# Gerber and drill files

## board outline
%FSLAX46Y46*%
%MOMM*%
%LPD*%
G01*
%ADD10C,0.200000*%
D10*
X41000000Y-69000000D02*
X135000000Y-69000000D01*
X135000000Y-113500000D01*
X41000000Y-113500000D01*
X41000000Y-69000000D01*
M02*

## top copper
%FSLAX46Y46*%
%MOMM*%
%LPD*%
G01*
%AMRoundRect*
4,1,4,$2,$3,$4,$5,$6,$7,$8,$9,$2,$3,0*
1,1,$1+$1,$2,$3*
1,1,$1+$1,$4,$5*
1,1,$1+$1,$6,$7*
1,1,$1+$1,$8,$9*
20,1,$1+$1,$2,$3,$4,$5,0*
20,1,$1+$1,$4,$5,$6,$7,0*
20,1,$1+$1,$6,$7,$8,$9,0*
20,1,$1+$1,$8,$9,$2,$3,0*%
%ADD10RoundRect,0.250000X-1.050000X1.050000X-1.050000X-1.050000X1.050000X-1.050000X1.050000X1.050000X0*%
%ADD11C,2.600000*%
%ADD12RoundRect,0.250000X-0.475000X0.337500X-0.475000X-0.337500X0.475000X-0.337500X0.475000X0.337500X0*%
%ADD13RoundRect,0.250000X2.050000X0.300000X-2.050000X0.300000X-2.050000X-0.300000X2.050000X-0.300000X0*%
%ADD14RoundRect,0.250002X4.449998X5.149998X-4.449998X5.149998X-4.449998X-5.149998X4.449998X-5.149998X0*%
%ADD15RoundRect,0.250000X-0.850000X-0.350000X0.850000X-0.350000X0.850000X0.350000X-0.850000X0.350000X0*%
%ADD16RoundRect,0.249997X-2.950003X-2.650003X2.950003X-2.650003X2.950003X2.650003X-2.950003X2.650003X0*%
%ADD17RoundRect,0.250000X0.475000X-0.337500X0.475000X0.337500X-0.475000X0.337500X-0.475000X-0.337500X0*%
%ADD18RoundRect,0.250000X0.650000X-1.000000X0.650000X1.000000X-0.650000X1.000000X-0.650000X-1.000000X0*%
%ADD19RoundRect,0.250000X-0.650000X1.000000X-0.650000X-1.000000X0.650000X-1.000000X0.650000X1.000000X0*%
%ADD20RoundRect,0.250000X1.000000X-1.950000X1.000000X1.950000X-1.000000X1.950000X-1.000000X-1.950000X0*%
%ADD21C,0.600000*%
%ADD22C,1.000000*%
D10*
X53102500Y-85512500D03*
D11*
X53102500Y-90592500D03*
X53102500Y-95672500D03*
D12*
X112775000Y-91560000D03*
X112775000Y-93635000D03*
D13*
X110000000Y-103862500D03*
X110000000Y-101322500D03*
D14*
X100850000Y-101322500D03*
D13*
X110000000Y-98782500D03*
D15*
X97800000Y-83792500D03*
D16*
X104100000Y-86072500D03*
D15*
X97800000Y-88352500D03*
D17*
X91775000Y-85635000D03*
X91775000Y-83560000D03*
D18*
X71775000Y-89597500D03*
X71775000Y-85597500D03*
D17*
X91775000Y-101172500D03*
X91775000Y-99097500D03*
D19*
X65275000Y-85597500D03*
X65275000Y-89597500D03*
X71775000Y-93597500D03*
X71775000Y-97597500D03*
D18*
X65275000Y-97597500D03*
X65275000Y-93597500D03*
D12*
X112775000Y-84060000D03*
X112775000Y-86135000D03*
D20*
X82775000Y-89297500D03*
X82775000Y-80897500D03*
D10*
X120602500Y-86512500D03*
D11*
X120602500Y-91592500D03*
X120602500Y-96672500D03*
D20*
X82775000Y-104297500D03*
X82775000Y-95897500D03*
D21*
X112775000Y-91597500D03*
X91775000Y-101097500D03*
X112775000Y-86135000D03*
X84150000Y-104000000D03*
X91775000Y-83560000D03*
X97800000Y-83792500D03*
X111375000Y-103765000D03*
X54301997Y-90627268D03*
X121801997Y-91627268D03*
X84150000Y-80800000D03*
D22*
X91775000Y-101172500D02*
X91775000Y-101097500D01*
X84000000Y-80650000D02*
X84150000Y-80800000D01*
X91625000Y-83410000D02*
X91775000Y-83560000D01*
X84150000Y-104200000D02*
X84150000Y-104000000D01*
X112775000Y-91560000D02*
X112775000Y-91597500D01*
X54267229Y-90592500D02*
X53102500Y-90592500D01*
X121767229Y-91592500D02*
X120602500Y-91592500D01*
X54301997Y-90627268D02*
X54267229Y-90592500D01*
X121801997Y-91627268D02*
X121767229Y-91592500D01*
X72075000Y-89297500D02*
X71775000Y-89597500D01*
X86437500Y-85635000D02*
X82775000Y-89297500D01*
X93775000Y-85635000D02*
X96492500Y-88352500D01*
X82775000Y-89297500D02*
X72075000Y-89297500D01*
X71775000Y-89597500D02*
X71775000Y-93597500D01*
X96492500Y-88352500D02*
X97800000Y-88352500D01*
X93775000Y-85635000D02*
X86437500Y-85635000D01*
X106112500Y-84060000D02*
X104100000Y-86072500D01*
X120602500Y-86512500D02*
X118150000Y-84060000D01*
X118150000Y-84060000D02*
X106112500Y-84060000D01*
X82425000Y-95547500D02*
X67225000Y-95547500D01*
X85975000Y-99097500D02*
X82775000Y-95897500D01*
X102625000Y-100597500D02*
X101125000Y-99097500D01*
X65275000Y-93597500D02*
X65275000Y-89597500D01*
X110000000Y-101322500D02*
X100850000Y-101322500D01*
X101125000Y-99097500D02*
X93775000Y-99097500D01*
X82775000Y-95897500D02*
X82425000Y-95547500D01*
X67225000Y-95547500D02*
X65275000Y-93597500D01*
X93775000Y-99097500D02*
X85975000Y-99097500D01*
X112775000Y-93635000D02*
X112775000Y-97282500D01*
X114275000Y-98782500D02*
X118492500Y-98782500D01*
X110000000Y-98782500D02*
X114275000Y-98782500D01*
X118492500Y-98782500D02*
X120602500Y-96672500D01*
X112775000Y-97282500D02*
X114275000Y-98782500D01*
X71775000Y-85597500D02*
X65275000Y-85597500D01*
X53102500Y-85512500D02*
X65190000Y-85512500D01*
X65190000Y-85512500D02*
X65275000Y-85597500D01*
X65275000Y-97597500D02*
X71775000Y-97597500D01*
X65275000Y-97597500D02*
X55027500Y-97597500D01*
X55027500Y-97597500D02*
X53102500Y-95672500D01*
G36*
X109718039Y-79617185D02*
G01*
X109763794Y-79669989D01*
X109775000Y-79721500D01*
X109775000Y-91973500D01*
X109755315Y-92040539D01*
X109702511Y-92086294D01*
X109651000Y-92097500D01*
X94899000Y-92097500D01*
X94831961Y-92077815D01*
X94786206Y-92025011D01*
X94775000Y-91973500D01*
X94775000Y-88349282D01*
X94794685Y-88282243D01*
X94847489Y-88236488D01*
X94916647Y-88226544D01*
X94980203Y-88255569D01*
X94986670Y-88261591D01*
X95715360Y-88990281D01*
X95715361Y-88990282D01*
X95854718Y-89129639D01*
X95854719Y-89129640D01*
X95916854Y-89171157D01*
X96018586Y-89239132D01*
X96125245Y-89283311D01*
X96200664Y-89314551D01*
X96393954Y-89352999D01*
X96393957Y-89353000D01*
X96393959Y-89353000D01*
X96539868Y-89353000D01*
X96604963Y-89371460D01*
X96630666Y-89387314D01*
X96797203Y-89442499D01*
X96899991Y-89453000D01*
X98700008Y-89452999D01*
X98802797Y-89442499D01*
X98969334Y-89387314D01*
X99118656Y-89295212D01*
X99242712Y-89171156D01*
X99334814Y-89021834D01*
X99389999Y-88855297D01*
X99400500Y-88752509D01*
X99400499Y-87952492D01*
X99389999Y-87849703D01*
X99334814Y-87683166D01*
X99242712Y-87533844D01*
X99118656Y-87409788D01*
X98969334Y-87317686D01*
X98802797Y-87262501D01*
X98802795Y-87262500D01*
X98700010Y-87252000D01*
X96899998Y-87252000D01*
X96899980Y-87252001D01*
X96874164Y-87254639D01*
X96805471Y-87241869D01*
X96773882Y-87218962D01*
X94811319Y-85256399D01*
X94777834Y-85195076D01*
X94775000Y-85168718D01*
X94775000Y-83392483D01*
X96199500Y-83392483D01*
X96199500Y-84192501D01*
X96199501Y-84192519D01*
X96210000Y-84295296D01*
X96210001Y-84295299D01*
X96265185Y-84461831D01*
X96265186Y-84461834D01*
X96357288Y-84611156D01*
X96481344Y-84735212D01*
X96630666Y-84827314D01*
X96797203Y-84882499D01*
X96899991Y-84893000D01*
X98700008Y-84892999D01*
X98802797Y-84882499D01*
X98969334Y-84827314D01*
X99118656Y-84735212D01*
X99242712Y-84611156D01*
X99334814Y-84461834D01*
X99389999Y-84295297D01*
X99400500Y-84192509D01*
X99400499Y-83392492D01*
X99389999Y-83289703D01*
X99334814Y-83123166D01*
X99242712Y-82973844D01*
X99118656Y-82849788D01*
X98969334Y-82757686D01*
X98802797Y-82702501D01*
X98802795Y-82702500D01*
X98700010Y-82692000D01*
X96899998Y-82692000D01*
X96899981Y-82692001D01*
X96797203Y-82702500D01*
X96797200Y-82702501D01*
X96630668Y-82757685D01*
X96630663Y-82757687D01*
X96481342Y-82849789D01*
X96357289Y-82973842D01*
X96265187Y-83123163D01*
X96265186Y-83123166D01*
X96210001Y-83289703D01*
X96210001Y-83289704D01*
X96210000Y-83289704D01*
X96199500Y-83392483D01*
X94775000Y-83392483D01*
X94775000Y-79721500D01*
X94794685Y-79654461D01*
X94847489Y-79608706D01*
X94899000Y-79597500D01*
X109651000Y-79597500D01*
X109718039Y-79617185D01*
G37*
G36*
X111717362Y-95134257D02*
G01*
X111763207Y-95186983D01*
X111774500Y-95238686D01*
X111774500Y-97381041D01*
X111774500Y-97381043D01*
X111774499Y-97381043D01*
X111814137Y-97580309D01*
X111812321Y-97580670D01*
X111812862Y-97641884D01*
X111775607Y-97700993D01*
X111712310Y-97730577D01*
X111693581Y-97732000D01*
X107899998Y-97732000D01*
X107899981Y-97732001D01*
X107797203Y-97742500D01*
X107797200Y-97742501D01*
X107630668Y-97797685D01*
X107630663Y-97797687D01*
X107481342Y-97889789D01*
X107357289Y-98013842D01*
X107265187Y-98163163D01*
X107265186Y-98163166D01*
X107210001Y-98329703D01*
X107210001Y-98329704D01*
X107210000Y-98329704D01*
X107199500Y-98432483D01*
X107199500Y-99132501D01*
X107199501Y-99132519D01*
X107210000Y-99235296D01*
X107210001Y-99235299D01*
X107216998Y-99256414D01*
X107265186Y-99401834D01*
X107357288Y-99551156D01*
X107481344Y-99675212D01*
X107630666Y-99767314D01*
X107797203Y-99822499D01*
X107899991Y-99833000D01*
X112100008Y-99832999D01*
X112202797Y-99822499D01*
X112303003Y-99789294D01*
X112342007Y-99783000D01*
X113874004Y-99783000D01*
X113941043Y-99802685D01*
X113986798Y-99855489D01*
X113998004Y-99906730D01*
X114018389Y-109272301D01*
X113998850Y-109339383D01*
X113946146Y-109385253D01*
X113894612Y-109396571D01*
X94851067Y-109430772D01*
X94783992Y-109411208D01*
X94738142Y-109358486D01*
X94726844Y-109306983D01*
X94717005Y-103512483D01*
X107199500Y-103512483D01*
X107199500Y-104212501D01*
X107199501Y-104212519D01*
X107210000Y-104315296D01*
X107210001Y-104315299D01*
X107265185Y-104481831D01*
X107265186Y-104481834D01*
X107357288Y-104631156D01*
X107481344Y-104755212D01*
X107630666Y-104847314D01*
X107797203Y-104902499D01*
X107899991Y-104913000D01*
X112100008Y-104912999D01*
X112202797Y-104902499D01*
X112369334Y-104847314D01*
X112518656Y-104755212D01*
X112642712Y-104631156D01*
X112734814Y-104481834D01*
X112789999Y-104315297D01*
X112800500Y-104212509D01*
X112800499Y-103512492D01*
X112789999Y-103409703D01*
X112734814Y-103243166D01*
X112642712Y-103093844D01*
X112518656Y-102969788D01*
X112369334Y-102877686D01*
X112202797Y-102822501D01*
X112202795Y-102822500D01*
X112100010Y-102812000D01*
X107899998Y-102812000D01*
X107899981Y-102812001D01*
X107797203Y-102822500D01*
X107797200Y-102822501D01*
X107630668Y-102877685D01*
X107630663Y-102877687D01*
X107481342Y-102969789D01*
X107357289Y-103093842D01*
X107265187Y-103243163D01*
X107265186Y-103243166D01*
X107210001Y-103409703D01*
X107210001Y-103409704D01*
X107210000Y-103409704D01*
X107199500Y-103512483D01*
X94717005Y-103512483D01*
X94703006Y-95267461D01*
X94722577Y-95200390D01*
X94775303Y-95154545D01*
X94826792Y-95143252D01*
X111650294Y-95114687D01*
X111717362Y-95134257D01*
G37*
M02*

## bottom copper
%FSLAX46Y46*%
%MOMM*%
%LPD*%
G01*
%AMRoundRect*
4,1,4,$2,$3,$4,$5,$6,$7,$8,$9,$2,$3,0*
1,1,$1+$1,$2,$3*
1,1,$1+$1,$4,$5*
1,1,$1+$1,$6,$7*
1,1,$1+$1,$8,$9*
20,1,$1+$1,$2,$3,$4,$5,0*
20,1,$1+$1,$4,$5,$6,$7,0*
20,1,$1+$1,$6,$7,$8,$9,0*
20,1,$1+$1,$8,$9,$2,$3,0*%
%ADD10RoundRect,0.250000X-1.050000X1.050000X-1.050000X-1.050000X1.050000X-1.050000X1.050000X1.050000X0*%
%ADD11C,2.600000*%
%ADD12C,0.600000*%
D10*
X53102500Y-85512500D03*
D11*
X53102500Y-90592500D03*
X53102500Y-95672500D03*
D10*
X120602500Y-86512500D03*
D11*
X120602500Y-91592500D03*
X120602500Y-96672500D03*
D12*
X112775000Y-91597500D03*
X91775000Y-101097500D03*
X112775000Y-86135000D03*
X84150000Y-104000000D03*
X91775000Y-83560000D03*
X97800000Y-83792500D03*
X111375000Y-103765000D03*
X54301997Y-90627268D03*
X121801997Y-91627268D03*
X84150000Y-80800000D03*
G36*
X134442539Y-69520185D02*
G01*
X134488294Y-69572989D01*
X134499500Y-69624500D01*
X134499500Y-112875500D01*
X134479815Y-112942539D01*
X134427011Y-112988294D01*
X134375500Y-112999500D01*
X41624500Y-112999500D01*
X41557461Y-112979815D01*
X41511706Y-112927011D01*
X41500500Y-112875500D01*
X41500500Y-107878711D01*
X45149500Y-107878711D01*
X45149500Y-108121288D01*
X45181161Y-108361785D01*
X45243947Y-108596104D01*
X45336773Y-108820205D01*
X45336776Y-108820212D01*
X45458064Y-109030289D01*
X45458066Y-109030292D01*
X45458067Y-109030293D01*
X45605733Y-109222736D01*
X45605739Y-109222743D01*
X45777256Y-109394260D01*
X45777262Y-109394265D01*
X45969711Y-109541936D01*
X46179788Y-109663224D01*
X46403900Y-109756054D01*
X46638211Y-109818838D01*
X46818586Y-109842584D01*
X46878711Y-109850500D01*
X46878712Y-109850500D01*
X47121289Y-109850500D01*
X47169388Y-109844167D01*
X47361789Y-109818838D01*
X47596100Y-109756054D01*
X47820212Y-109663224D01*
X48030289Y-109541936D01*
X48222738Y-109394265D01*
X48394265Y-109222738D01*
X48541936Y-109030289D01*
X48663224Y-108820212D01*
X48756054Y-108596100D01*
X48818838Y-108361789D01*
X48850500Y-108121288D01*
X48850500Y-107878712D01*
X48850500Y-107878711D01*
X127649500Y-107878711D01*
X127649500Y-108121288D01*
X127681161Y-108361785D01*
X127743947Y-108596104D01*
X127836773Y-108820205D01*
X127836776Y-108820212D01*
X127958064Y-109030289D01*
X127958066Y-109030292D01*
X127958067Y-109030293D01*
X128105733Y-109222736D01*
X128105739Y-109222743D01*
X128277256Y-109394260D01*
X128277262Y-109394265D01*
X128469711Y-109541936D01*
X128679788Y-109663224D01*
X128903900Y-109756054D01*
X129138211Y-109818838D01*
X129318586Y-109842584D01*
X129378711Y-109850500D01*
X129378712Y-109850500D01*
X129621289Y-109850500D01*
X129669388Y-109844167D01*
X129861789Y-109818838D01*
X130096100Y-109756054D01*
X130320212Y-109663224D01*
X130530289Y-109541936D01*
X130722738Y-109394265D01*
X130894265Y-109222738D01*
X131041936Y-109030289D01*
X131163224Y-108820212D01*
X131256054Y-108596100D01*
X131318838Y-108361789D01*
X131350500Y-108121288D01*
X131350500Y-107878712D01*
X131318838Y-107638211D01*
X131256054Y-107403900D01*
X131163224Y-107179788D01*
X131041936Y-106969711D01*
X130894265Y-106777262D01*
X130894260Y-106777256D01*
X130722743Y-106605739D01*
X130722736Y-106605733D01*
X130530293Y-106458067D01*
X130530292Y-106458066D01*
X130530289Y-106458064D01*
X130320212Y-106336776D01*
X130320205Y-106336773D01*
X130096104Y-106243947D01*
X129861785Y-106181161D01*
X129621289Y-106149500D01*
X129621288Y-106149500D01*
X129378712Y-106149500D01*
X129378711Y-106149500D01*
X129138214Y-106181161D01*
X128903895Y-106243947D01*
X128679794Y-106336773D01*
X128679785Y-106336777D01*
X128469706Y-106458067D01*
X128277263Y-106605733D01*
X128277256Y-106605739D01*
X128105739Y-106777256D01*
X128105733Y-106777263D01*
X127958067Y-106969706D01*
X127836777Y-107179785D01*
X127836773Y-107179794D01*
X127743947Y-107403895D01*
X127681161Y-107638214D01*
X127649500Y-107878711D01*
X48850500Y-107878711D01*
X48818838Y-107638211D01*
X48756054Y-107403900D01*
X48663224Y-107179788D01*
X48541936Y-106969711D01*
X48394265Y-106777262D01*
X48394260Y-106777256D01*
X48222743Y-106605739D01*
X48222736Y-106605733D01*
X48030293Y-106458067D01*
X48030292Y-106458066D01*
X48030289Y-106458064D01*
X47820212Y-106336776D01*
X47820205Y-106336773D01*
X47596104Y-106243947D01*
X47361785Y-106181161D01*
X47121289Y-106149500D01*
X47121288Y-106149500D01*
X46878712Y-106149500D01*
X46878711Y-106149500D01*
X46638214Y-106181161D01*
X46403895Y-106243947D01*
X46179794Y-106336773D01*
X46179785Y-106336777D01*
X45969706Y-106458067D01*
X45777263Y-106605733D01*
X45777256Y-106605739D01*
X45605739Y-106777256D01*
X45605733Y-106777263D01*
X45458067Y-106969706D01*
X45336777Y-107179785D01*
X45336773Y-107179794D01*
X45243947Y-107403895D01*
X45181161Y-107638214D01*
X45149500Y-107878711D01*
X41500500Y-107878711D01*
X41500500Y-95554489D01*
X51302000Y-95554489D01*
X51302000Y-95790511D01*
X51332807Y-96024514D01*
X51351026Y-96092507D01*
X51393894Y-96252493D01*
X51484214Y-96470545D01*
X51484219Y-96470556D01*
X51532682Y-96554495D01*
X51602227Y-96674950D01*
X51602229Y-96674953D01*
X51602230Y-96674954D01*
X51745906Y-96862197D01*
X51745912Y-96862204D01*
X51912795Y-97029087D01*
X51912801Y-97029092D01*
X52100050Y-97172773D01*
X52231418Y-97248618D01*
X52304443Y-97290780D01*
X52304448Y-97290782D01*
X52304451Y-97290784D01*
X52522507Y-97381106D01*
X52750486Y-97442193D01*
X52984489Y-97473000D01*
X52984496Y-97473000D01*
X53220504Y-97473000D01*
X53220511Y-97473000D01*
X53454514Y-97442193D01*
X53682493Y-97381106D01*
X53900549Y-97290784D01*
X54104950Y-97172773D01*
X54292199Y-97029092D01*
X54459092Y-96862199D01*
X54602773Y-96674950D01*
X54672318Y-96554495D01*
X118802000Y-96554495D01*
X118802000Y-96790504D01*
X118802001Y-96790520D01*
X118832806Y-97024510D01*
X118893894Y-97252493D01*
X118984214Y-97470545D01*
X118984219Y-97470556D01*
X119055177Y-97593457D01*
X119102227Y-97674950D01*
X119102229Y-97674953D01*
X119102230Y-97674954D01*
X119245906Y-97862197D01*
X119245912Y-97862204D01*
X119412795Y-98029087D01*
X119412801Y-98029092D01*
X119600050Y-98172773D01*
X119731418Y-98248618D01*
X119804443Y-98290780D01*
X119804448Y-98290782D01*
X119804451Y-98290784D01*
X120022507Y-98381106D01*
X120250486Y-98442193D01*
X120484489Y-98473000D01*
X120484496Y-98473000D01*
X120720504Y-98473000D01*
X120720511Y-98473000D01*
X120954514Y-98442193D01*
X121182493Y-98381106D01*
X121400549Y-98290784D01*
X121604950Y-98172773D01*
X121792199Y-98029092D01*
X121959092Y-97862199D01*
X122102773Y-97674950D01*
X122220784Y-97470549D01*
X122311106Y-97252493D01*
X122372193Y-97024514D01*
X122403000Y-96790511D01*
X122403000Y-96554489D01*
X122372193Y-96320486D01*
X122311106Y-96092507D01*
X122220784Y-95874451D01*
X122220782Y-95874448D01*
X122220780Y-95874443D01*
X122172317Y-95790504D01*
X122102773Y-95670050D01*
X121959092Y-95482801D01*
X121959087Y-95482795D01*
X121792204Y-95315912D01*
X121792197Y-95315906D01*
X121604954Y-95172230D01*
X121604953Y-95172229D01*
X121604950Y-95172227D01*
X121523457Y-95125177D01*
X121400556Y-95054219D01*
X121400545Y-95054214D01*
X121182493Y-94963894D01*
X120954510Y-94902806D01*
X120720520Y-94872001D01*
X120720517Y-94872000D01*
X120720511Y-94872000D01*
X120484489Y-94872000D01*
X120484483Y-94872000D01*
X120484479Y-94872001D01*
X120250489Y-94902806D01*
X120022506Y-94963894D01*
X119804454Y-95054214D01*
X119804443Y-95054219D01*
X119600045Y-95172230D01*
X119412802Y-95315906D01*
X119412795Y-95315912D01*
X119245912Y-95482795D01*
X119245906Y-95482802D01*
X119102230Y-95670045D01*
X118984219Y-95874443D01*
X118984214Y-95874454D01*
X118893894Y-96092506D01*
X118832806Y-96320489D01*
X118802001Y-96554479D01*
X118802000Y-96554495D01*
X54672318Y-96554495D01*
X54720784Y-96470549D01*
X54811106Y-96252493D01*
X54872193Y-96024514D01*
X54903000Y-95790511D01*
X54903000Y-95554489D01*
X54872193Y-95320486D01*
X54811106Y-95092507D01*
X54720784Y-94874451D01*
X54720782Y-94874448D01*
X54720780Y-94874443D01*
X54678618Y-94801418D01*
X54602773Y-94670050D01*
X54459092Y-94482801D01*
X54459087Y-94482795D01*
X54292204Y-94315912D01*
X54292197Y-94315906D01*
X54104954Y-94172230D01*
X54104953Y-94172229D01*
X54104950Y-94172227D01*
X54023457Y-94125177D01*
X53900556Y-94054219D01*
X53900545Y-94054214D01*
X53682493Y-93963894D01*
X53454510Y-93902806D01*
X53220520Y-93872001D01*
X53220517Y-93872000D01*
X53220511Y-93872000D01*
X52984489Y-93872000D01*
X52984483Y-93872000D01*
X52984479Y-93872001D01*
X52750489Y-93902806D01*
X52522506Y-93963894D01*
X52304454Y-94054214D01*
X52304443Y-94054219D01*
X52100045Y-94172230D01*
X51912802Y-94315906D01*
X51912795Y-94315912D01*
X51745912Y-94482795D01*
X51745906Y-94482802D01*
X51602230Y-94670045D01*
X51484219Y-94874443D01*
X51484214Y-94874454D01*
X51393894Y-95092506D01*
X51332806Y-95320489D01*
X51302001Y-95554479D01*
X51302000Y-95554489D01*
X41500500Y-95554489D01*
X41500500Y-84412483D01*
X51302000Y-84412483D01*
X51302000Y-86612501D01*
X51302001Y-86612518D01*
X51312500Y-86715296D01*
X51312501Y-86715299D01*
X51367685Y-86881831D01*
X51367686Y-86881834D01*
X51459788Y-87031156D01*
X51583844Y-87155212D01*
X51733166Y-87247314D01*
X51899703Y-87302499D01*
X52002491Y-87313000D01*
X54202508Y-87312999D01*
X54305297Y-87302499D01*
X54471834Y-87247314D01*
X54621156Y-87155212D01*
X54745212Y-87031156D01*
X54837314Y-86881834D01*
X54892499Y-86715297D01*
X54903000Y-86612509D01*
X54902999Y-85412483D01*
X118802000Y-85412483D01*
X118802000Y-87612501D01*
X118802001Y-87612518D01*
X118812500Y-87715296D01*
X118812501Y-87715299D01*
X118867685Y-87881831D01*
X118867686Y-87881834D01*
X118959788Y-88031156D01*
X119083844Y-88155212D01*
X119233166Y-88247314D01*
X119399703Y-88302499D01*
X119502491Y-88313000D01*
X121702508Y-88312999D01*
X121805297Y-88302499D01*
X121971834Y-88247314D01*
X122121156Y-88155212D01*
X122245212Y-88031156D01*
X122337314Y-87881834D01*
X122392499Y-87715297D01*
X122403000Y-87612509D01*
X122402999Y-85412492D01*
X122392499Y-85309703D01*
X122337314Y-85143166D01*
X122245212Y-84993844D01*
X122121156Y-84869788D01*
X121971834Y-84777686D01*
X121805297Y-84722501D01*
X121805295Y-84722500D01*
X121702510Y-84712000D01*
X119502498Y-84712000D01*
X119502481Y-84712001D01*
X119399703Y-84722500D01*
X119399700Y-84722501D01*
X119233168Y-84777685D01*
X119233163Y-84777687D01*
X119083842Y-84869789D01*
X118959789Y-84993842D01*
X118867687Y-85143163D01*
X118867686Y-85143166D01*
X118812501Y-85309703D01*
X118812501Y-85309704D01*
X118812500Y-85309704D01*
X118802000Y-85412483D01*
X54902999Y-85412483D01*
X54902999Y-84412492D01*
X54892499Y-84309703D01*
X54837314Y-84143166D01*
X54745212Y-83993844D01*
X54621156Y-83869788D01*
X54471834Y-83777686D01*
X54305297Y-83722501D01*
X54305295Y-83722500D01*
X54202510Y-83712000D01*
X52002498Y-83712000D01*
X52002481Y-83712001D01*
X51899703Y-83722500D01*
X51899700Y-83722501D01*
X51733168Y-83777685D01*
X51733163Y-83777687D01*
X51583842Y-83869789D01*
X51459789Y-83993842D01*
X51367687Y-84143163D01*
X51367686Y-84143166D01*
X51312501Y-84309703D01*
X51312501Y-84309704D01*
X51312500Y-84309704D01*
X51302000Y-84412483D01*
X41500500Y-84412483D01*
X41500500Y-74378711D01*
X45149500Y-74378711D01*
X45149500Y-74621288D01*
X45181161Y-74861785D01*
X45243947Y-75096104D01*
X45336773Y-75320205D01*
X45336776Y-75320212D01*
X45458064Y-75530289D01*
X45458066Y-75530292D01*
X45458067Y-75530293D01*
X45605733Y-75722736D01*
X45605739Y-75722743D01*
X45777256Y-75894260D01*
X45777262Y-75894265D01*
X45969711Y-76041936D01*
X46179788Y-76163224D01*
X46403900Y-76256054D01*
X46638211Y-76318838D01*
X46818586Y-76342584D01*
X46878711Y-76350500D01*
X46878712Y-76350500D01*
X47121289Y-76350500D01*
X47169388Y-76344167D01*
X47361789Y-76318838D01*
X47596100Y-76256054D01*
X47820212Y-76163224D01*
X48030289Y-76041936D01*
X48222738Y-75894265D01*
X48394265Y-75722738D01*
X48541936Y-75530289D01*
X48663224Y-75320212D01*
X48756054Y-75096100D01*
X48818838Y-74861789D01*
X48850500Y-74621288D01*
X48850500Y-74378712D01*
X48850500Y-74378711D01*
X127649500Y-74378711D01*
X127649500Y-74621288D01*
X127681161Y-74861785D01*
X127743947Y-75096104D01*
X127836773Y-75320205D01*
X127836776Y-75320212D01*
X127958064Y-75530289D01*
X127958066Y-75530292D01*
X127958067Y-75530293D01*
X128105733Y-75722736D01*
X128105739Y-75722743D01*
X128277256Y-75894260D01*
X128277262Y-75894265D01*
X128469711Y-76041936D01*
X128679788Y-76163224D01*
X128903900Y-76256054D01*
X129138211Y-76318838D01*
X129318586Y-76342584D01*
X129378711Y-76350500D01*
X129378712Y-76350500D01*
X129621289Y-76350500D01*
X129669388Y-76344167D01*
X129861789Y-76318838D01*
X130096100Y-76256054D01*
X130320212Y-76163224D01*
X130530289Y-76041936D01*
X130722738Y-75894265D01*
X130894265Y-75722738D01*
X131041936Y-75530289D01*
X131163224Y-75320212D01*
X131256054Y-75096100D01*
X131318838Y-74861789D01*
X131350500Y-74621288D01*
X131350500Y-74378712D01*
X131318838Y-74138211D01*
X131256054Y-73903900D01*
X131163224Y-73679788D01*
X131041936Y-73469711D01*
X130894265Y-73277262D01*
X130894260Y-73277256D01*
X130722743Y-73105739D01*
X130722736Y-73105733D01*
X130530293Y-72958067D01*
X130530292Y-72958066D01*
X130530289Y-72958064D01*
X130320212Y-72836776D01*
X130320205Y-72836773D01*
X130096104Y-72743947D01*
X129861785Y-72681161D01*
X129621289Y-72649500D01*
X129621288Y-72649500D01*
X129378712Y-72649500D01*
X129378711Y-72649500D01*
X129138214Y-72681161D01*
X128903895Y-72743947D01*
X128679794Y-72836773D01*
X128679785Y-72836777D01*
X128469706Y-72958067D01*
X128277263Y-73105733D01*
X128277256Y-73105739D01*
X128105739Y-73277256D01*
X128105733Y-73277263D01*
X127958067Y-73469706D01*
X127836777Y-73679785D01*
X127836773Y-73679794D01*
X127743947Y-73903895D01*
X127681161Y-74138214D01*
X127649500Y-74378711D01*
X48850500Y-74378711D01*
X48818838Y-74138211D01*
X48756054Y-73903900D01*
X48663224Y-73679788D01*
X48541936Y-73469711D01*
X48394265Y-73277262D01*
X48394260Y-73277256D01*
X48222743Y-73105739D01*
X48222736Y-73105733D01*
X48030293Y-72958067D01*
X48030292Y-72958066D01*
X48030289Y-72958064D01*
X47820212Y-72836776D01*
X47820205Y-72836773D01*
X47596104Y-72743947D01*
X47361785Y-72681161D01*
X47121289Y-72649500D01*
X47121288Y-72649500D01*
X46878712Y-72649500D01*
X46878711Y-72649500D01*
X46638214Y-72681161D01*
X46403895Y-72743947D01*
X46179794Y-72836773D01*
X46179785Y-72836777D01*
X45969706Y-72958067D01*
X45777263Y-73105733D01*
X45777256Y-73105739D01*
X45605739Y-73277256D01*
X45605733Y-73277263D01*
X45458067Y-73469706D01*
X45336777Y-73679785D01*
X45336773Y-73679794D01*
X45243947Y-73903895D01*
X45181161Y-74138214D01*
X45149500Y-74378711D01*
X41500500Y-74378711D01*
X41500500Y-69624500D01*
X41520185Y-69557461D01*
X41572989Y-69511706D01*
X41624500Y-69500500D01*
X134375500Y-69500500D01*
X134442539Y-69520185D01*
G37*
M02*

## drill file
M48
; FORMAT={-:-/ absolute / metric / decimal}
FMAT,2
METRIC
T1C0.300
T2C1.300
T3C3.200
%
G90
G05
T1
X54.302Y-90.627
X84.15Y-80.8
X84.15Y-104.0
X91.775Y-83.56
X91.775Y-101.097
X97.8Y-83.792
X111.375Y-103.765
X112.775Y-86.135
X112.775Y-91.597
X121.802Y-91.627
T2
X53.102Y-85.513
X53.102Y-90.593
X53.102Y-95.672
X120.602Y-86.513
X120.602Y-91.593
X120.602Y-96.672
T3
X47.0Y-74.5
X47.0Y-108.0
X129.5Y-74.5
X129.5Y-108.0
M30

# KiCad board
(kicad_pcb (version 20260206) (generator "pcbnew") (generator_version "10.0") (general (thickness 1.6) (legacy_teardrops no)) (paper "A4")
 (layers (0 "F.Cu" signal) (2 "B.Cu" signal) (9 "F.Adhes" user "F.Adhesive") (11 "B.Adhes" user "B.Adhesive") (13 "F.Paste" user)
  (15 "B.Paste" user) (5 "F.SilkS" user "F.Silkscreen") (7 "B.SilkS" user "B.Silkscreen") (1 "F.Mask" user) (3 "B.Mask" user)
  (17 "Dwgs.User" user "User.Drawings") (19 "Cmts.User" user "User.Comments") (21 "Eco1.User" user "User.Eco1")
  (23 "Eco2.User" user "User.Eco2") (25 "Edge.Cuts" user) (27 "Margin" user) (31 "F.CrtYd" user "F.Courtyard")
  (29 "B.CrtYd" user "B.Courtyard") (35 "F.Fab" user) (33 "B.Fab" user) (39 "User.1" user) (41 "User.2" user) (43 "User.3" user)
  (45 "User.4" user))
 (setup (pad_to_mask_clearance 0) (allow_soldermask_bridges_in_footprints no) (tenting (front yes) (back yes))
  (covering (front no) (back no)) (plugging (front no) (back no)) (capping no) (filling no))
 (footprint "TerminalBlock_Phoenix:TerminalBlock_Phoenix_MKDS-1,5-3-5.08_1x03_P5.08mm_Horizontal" (layer "F.Cu") (at 53.1025 85.5125 -90)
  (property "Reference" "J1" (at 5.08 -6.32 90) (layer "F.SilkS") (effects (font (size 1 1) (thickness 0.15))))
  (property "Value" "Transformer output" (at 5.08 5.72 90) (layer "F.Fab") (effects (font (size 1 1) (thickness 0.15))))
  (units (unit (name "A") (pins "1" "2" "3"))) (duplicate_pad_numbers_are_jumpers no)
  (pad "1" thru_hole roundrect (at 0 0 270) (size 2.6 2.6) (drill 1.3) (layers "*.Cu" "*.Mask") (remove_unused_layers no)
   (roundrect_rratio 0.096154) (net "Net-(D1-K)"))
  (pad "2" thru_hole circle (at 5.08 0 270) (size 2.6 2.6) (drill 1.3) (layers "*.Cu" "*.Mask") (remove_unused_layers no) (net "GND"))
  (pad "3" thru_hole circle (at 10.16 0 270) (size 2.6 2.6) (drill 1.3) (layers "*.Cu" "*.Mask") (remove_unused_layers no)
   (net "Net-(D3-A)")))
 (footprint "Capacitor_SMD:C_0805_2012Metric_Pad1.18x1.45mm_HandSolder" (layer "F.Cu") (at 112.775 92.5975 -90)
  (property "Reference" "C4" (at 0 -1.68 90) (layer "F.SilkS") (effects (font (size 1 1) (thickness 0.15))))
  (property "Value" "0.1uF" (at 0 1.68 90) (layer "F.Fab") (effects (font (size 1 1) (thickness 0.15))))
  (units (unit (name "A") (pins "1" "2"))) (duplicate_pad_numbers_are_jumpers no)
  (pad "1" smd roundrect (at -1.0375 0 270) (size 1.175 1.45) (layers "F.Cu" "F.Mask" "F.Paste") (roundrect_rratio 0.212766) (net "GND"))
  (pad "2" smd roundrect (at 1.0375 0 270) (size 1.175 1.45) (layers "F.Cu" "F.Mask" "F.Paste") (roundrect_rratio 0.212766)
   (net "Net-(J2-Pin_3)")))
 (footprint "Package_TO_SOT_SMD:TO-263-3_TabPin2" (layer "F.Cu") (at 102.35 101.3225 180)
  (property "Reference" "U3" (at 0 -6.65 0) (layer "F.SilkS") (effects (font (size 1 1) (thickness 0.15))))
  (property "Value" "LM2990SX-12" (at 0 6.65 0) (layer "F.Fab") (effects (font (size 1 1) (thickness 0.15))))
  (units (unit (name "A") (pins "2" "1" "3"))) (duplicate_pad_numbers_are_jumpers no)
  (pad "" smd roundrect (at -0.925 -2.775 180) (size 4.55 5.25) (layers "F.Paste") (roundrect_rratio 0.054945))
  (pad "" smd roundrect (at -0.925 2.775 180) (size 4.55 5.25) (layers "F.Paste") (roundrect_rratio 0.054945))
  (pad "" smd roundrect (at 3.925 -2.775 180) (size 4.55 5.25) (layers "F.Paste") (roundrect_rratio 0.054945))
  (pad "" smd roundrect (at 3.925 2.775 180) (size 4.55 5.25) (layers "F.Paste") (roundrect_rratio 0.054945))
  (pad "1" smd roundrect (at -7.65 -2.54 180) (size 4.6 1.1) (layers "F.Cu" "F.Mask" "F.Paste") (roundrect_rratio 0.227273) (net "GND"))
  (pad "2" smd roundrect (at -7.65 0 180) (size 4.6 1.1) (layers "F.Cu" "F.Mask" "F.Paste") (roundrect_rratio 0.227273) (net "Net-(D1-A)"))
  (pad "2" smd roundrect (at 1.5 0 180) (size 9.4 10.8) (layers "F.Cu" "F.Mask") (roundrect_rratio 0.026596) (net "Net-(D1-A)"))
  (pad "3" smd roundrect (at -7.65 2.54 180) (size 4.6 1.1) (layers "F.Cu" "F.Mask" "F.Paste") (roundrect_rratio 0.227273)
   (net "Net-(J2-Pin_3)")))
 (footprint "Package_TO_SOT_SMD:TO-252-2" (layer "F.Cu") (at 102.84 86.0725)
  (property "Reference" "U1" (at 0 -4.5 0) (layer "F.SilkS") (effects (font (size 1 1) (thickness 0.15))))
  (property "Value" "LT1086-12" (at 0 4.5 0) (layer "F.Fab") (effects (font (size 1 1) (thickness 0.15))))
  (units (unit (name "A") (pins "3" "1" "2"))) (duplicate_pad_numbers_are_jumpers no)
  (pad "" smd roundrect (at -0.415 -1.525) (size 3.05 2.75) (layers "F.Paste") (roundrect_rratio 0.090909))
  (pad "" smd roundrect (at -0.415 1.525) (size 3.05 2.75) (layers "F.Paste") (roundrect_rratio 0.090909))
  (pad "" smd roundrect (at 2.935 -1.525) (size 3.05 2.75) (layers "F.Paste") (roundrect_rratio 0.090909))
  (pad "" smd roundrect (at 2.935 1.525) (size 3.05 2.75) (layers "F.Paste") (roundrect_rratio 0.090909))
  (pad "1" smd roundrect (at -5.04 -2.28) (size 2.2 1.2) (layers "F.Cu" "F.Mask" "F.Paste") (roundrect_rratio 0.208333) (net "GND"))
  (pad "2" smd roundrect (at 1.26 0) (size 6.4 5.8) (layers "F.Cu" "F.Mask") (roundrect_rratio 0.043103) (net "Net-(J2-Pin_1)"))
  (pad "3" smd roundrect (at -5.04 2.28) (size 2.2 1.2) (layers "F.Cu" "F.Mask" "F.Paste") (roundrect_rratio 0.208333) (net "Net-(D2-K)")))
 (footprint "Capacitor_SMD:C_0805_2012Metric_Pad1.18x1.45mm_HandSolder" (layer "F.Cu") (at 91.775 84.5975 90)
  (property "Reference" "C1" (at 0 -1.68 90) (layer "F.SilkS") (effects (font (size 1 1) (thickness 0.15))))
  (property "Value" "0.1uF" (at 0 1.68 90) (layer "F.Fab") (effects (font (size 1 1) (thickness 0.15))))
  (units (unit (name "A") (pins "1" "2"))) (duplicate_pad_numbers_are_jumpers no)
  (pad "1" smd roundrect (at -1.0375 0 90) (size 1.175 1.45) (layers "F.Cu" "F.Mask" "F.Paste") (roundrect_rratio 0.212766)
   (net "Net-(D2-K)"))
  (pad "2" smd roundrect (at 1.0375 0 90) (size 1.175 1.45) (layers "F.Cu" "F.Mask" "F.Paste") (roundrect_rratio 0.212766) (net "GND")))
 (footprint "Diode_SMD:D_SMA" (layer "F.Cu") (at 71.775 87.5975 90)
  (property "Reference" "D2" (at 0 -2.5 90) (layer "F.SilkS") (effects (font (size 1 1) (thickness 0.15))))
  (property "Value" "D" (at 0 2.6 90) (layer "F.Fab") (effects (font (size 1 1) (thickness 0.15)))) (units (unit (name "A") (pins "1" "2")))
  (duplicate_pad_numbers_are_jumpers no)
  (pad "1" smd roundrect (at -2 0 90) (size 2.5 1.8) (layers "F.Cu" "F.Mask" "F.Paste") (roundrect_rratio 0.1388888889) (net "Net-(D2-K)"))
  (pad "2" smd roundrect (at 2 0 90) (size 2.5 1.8) (layers "F.Cu" "F.Mask" "F.Paste") (roundrect_rratio 0.1388888889) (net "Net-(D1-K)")))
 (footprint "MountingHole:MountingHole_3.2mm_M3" (layer "F.Cu") (at 47 74.5)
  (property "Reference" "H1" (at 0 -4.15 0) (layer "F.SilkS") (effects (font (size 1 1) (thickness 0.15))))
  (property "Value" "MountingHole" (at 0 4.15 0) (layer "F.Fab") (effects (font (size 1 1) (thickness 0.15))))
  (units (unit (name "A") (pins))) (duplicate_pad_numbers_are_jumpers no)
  (pad "" np_thru_hole circle (at 0 0) (size 3.2 3.2) (drill 3.2) (layers "*.Cu" "*.Mask")))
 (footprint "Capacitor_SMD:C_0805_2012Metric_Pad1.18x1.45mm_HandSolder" (layer "F.Cu") (at 91.775 100.135 90)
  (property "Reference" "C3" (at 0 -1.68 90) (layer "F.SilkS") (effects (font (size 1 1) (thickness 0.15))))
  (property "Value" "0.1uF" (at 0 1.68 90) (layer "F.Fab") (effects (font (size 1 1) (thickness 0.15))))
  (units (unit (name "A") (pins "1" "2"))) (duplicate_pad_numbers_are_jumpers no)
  (pad "1" smd roundrect (at -1.0375 0 90) (size 1.175 1.45) (layers "F.Cu" "F.Mask" "F.Paste") (roundrect_rratio 0.212766) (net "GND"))
  (pad "2" smd roundrect (at 1.0375 0 90) (size 1.175 1.45) (layers "F.Cu" "F.Mask" "F.Paste") (roundrect_rratio 0.212766)
   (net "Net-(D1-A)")))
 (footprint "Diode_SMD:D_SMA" (layer "F.Cu") (at 65.275 87.5975 -90)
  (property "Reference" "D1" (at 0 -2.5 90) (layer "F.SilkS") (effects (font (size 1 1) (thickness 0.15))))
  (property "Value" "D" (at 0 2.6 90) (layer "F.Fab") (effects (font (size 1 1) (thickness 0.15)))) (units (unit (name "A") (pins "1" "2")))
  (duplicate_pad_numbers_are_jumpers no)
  (pad "1" smd roundrect (at -2 0 270) (size 2.5 1.8) (layers "F.Cu" "F.Mask" "F.Paste") (roundrect_rratio 0.1388888889) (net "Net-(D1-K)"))
  (pad "2" smd roundrect (at 2 0 270) (size 2.5 1.8) (layers "F.Cu" "F.Mask" "F.Paste") (roundrect_rratio 0.1388888889) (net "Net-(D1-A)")))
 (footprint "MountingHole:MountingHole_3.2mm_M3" (layer "F.Cu") (at 47 108)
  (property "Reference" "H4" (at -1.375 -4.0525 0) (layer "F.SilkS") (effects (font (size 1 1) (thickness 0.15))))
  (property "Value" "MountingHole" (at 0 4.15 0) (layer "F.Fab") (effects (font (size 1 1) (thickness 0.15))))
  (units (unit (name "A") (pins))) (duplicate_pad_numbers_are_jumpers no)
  (pad "" np_thru_hole circle (at 0 0) (size 3.2 3.2) (drill 3.2) (layers "*.Cu" "*.Mask")))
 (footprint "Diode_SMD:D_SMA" (layer "F.Cu") (at 71.775 95.5975 -90)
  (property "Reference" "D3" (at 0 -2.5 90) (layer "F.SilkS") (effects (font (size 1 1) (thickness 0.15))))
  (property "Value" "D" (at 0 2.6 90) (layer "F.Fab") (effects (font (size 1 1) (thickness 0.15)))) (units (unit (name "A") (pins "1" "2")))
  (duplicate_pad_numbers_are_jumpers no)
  (pad "1" smd roundrect (at -2 0 270) (size 2.5 1.8) (layers "F.Cu" "F.Mask" "F.Paste") (roundrect_rratio 0.1388888889) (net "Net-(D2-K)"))
  (pad "2" smd roundrect (at 2 0 270) (size 2.5 1.8) (layers "F.Cu" "F.Mask" "F.Paste") (roundrect_rratio 0.1388888889) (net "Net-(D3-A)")))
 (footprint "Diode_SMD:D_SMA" (layer "F.Cu") (at 65.275 95.5975 90)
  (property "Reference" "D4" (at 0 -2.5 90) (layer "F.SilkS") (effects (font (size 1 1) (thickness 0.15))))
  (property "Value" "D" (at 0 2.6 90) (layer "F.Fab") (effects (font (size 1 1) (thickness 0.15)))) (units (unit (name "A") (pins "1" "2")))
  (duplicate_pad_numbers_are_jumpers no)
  (pad "1" smd roundrect (at -2 0 90) (size 2.5 1.8) (layers "F.Cu" "F.Mask" "F.Paste") (roundrect_rratio 0.1388888889) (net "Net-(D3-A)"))
  (pad "2" smd roundrect (at 2 0 90) (size 2.5 1.8) (layers "F.Cu" "F.Mask" "F.Paste") (roundrect_rratio 0.1388888889) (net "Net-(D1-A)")))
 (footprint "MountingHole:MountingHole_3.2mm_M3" (layer "F.Cu") (at 129.5 108)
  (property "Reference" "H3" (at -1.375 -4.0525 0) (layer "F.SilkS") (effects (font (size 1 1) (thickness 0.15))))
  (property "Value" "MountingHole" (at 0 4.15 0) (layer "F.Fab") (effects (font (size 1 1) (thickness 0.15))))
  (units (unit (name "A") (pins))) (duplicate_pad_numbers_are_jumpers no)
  (pad "" np_thru_hole circle (at 0 0) (size 3.2 3.2) (drill 3.2) (layers "*.Cu" "*.Mask")))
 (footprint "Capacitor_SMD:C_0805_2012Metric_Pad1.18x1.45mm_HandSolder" (layer "F.Cu") (at 112.775 85.0975 -90)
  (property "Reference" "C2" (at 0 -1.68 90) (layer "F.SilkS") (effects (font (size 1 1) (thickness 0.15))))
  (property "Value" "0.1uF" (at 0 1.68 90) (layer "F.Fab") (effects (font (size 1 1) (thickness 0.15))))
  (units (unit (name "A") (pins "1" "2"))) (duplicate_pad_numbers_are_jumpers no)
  (pad "1" smd roundrect (at -1.0375 0 270) (size 1.175 1.45) (layers "F.Cu" "F.Mask" "F.Paste") (roundrect_rratio 0.212766)
   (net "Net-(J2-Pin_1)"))
  (pad "2" smd roundrect (at 1.0375 0 270) (size 1.175 1.45) (layers "F.Cu" "F.Mask" "F.Paste") (roundrect_rratio 0.212766) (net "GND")))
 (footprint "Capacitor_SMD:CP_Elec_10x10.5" (layer "F.Cu") (at 82.775 85.0975 90)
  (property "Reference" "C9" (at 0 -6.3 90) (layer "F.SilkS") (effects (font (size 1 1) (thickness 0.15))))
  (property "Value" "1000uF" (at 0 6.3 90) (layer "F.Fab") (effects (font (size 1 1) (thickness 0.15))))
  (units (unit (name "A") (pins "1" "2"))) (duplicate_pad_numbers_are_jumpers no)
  (pad "1" smd roundrect (at -4.2 0 90) (size 4.4 2.5) (layers "F.Cu" "F.Mask" "F.Paste") (roundrect_rratio 0.1) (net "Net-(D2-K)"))
  (pad "2" smd roundrect (at 4.2 0 90) (size 4.4 2.5) (layers "F.Cu" "F.Mask" "F.Paste") (roundrect_rratio 0.1) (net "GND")))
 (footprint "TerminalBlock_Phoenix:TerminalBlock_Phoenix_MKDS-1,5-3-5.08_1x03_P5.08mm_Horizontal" (layer "F.Cu") (at 120.6025 86.5125 -90)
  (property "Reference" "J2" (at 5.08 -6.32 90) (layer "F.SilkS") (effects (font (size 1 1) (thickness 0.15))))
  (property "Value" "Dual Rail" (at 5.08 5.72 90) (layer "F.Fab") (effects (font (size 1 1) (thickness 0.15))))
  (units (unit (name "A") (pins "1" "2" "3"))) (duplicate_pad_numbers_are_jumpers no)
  (pad "1" thru_hole roundrect (at 0 0 270) (size 2.6 2.6) (drill 1.3) (layers "*.Cu" "*.Mask") (remove_unused_layers no)
   (roundrect_rratio 0.096154) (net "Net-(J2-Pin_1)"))
  (pad "2" thru_hole circle (at 5.08 0 270) (size 2.6 2.6) (drill 1.3) (layers "*.Cu" "*.Mask") (remove_unused_layers no) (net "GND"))
  (pad "3" thru_hole circle (at 10.16 0 270) (size 2.6 2.6) (drill 1.3) (layers "*.Cu" "*.Mask") (remove_unused_layers no)
   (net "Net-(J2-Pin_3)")))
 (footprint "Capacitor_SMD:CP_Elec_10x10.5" (layer "F.Cu") (at 82.775 100.0975 90)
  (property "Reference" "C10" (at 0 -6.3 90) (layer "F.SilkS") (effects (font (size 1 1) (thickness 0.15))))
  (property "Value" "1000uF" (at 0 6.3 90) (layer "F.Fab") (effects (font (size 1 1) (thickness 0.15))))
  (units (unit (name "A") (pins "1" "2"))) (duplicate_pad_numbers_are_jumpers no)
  (pad "1" smd roundrect (at -4.2 0 90) (size 4.4 2.5) (layers "F.Cu" "F.Mask" "F.Paste") (roundrect_rratio 0.1) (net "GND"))
  (pad "2" smd roundrect (at 4.2 0 90) (size 4.4 2.5) (layers "F.Cu" "F.Mask" "F.Paste") (roundrect_rratio 0.1) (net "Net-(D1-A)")))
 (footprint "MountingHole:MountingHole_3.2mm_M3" (layer "F.Cu") (at 129.5 74.5)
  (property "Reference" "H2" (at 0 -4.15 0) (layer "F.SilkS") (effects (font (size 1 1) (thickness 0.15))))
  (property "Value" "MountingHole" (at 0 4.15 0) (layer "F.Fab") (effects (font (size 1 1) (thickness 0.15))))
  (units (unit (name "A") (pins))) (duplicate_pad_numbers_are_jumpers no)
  (pad "" np_thru_hole circle (at 0 0) (size 3.2 3.2) (drill 3.2) (layers "*.Cu" "*.Mask")))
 (gr_rect (start 41 69) (end 135 113.5) (stroke (width 0.2) (type solid)) (fill no) (layer "Edge.Cuts"))
 (segment (start 71.775 85.5975) (end 65.275 85.5975) (width 1) (layer "F.Cu") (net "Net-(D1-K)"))
 (segment (start 53.1025 85.5125) (end 65.19 85.5125) (width 1) (layer "F.Cu") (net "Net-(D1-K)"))
 (segment (start 65.19 85.5125) (end 65.275 85.5975) (width 1) (layer "F.Cu") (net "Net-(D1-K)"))
 (segment (start 91.775 101.1725) (end 91.775 101.0975) (width 1) (layer "F.Cu") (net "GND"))
 (segment (start 84 80.65) (end 84.15 80.8) (width 1) (layer "F.Cu") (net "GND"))
 (segment (start 91.625 83.41) (end 91.775 83.56) (width 1) (layer "F.Cu") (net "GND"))
 (segment (start 84.15 104.2) (end 84.15 104) (width 1) (layer "F.Cu") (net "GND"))
 (segment (start 112.775 91.56) (end 112.775 91.5975) (width 1) (layer "F.Cu") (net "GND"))
 (segment (start 54.267229 90.5925) (end 53.1025 90.5925) (width 1) (layer "F.Cu") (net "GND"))
 (segment (start 121.767229 91.5925) (end 120.6025 91.5925) (width 1) (layer "F.Cu") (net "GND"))
 (segment (start 54.301997 90.627268) (end 54.267229 90.5925) (width 1) (layer "F.Cu") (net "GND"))
 (segment (start 121.801997 91.627268) (end 121.767229 91.5925) (width 1) (layer "F.Cu") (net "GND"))
 (via (at 112.775 91.5975) (size 0.6) (drill 0.3) (layers "F.Cu" "B.Cu") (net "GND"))
 (via (at 91.775 101.0975) (size 0.6) (drill 0.3) (layers "F.Cu" "B.Cu") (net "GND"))
 (via (at 112.775 86.135) (size 0.6) (drill 0.3) (layers "F.Cu" "B.Cu") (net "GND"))
 (via (at 84.15 104) (size 0.6) (drill 0.3) (layers "F.Cu" "B.Cu") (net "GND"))
 (via (at 91.775 83.56) (size 0.6) (drill 0.3) (layers "F.Cu" "B.Cu") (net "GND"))
 (via (at 97.8 83.7925) (size 0.6) (drill 0.3) (layers "F.Cu" "B.Cu") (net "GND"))
 (via (at 111.375 103.765) (size 0.6) (drill 0.3) (layers "F.Cu" "B.Cu") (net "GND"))
 (via (at 54.301997 90.627268) (size 0.6) (drill 0.3) (layers "F.Cu" "B.Cu") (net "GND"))
 (via (at 121.801997 91.627268) (size 0.6) (drill 0.3) (layers "F.Cu" "B.Cu") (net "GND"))
 (via (at 84.15 80.8) (size 0.6) (drill 0.3) (layers "F.Cu" "B.Cu") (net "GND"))
 (segment (start 65.275 97.5975) (end 71.775 97.5975) (width 1) (layer "F.Cu") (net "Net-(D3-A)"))
 (segment (start 65.275 97.5975) (end 55.0275 97.5975) (width 1) (layer "F.Cu") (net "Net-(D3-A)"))
 (segment (start 55.0275 97.5975) (end 53.1025 95.6725) (width 1) (layer "F.Cu") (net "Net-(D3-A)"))
 (segment (start 112.775 93.635) (end 112.775 97.2825) (width 1) (layer "F.Cu") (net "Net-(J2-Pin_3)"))
 (segment (start 114.275 98.7825) (end 118.4925 98.7825) (width 1) (layer "F.Cu") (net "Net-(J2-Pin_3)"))
 (segment (start 110 98.7825) (end 114.275 98.7825) (width 1) (layer "F.Cu") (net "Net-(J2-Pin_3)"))
 (segment (start 118.4925 98.7825) (end 120.6025 96.6725) (width 1) (layer "F.Cu") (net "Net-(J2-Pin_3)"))
 (segment (start 112.775 97.2825) (end 114.275 98.7825) (width 1) (layer "F.Cu") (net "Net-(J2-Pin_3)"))
 (segment (start 82.425 95.5475) (end 67.225 95.5475) (width 1) (layer "F.Cu") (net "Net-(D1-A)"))
 (segment (start 85.975 99.0975) (end 82.775 95.8975) (width 1) (layer "F.Cu") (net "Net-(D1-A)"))
 (segment (start 102.625 100.5975) (end 101.125 99.0975) (width 1) (layer "F.Cu") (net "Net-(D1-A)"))
 (segment (start 65.275 93.5975) (end 65.275 89.5975) (width 1) (layer "F.Cu") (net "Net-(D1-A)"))
 (segment (start 110 101.3225) (end 100.85 101.3225) (width 1) (layer "F.Cu") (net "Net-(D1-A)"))
 (segment (start 101.125 99.0975) (end 93.775 99.0975) (width 1) (layer "F.Cu") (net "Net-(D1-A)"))
 (segment (start 82.775 95.8975) (end 82.425 95.5475) (width 1) (layer "F.Cu") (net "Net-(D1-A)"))
 (segment (start 67.225 95.5475) (end 65.275 93.5975) (width 1) (layer "F.Cu") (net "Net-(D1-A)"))
 (segment (start 93.775 99.0975) (end 85.975 99.0975) (width 1) (layer "F.Cu") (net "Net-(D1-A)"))
 (segment (start 106.1125 84.06) (end 104.1 86.0725) (width 1) (layer "F.Cu") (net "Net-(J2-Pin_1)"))
 (segment (start 120.6025 86.5125) (end 118.15 84.06) (width 1) (layer "F.Cu") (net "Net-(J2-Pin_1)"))
 (segment (start 118.15 84.06) (end 106.1125 84.06) (width 1) (layer "F.Cu") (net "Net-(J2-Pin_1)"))
 (segment (start 72.075 89.2975) (end 71.775 89.5975) (width 1) (layer "F.Cu") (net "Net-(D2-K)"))
 (segment (start 86.4375 85.635) (end 82.775 89.2975) (width 1) (layer "F.Cu") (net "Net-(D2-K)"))
 (segment (start 93.775 85.635) (end 96.4925 88.3525) (width 1) (layer "F.Cu") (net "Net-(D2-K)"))
 (segment (start 82.775 89.2975) (end 72.075 89.2975) (width 1) (layer "F.Cu") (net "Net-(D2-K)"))
 (segment (start 71.775 89.5975) (end 71.775 93.5975) (width 1) (layer "F.Cu") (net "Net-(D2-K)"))
 (segment (start 96.4925 88.3525) (end 97.8 88.3525) (width 1) (layer "F.Cu") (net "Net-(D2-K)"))
 (segment (start 93.775 85.635) (end 86.4375 85.635) (width 1) (layer "F.Cu") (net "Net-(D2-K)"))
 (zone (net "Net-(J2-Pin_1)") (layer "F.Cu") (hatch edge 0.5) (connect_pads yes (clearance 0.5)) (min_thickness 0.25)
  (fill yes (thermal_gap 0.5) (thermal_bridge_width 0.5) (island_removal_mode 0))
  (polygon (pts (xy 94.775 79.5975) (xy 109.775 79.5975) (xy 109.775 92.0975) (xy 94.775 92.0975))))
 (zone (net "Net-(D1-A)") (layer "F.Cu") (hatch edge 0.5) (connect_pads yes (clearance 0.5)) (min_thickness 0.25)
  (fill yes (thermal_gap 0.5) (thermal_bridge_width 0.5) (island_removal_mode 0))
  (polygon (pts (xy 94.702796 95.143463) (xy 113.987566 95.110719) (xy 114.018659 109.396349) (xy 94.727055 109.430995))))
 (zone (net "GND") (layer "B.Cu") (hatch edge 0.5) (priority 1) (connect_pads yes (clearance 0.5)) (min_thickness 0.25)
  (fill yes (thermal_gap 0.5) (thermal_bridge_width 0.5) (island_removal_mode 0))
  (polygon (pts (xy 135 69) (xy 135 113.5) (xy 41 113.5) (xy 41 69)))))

